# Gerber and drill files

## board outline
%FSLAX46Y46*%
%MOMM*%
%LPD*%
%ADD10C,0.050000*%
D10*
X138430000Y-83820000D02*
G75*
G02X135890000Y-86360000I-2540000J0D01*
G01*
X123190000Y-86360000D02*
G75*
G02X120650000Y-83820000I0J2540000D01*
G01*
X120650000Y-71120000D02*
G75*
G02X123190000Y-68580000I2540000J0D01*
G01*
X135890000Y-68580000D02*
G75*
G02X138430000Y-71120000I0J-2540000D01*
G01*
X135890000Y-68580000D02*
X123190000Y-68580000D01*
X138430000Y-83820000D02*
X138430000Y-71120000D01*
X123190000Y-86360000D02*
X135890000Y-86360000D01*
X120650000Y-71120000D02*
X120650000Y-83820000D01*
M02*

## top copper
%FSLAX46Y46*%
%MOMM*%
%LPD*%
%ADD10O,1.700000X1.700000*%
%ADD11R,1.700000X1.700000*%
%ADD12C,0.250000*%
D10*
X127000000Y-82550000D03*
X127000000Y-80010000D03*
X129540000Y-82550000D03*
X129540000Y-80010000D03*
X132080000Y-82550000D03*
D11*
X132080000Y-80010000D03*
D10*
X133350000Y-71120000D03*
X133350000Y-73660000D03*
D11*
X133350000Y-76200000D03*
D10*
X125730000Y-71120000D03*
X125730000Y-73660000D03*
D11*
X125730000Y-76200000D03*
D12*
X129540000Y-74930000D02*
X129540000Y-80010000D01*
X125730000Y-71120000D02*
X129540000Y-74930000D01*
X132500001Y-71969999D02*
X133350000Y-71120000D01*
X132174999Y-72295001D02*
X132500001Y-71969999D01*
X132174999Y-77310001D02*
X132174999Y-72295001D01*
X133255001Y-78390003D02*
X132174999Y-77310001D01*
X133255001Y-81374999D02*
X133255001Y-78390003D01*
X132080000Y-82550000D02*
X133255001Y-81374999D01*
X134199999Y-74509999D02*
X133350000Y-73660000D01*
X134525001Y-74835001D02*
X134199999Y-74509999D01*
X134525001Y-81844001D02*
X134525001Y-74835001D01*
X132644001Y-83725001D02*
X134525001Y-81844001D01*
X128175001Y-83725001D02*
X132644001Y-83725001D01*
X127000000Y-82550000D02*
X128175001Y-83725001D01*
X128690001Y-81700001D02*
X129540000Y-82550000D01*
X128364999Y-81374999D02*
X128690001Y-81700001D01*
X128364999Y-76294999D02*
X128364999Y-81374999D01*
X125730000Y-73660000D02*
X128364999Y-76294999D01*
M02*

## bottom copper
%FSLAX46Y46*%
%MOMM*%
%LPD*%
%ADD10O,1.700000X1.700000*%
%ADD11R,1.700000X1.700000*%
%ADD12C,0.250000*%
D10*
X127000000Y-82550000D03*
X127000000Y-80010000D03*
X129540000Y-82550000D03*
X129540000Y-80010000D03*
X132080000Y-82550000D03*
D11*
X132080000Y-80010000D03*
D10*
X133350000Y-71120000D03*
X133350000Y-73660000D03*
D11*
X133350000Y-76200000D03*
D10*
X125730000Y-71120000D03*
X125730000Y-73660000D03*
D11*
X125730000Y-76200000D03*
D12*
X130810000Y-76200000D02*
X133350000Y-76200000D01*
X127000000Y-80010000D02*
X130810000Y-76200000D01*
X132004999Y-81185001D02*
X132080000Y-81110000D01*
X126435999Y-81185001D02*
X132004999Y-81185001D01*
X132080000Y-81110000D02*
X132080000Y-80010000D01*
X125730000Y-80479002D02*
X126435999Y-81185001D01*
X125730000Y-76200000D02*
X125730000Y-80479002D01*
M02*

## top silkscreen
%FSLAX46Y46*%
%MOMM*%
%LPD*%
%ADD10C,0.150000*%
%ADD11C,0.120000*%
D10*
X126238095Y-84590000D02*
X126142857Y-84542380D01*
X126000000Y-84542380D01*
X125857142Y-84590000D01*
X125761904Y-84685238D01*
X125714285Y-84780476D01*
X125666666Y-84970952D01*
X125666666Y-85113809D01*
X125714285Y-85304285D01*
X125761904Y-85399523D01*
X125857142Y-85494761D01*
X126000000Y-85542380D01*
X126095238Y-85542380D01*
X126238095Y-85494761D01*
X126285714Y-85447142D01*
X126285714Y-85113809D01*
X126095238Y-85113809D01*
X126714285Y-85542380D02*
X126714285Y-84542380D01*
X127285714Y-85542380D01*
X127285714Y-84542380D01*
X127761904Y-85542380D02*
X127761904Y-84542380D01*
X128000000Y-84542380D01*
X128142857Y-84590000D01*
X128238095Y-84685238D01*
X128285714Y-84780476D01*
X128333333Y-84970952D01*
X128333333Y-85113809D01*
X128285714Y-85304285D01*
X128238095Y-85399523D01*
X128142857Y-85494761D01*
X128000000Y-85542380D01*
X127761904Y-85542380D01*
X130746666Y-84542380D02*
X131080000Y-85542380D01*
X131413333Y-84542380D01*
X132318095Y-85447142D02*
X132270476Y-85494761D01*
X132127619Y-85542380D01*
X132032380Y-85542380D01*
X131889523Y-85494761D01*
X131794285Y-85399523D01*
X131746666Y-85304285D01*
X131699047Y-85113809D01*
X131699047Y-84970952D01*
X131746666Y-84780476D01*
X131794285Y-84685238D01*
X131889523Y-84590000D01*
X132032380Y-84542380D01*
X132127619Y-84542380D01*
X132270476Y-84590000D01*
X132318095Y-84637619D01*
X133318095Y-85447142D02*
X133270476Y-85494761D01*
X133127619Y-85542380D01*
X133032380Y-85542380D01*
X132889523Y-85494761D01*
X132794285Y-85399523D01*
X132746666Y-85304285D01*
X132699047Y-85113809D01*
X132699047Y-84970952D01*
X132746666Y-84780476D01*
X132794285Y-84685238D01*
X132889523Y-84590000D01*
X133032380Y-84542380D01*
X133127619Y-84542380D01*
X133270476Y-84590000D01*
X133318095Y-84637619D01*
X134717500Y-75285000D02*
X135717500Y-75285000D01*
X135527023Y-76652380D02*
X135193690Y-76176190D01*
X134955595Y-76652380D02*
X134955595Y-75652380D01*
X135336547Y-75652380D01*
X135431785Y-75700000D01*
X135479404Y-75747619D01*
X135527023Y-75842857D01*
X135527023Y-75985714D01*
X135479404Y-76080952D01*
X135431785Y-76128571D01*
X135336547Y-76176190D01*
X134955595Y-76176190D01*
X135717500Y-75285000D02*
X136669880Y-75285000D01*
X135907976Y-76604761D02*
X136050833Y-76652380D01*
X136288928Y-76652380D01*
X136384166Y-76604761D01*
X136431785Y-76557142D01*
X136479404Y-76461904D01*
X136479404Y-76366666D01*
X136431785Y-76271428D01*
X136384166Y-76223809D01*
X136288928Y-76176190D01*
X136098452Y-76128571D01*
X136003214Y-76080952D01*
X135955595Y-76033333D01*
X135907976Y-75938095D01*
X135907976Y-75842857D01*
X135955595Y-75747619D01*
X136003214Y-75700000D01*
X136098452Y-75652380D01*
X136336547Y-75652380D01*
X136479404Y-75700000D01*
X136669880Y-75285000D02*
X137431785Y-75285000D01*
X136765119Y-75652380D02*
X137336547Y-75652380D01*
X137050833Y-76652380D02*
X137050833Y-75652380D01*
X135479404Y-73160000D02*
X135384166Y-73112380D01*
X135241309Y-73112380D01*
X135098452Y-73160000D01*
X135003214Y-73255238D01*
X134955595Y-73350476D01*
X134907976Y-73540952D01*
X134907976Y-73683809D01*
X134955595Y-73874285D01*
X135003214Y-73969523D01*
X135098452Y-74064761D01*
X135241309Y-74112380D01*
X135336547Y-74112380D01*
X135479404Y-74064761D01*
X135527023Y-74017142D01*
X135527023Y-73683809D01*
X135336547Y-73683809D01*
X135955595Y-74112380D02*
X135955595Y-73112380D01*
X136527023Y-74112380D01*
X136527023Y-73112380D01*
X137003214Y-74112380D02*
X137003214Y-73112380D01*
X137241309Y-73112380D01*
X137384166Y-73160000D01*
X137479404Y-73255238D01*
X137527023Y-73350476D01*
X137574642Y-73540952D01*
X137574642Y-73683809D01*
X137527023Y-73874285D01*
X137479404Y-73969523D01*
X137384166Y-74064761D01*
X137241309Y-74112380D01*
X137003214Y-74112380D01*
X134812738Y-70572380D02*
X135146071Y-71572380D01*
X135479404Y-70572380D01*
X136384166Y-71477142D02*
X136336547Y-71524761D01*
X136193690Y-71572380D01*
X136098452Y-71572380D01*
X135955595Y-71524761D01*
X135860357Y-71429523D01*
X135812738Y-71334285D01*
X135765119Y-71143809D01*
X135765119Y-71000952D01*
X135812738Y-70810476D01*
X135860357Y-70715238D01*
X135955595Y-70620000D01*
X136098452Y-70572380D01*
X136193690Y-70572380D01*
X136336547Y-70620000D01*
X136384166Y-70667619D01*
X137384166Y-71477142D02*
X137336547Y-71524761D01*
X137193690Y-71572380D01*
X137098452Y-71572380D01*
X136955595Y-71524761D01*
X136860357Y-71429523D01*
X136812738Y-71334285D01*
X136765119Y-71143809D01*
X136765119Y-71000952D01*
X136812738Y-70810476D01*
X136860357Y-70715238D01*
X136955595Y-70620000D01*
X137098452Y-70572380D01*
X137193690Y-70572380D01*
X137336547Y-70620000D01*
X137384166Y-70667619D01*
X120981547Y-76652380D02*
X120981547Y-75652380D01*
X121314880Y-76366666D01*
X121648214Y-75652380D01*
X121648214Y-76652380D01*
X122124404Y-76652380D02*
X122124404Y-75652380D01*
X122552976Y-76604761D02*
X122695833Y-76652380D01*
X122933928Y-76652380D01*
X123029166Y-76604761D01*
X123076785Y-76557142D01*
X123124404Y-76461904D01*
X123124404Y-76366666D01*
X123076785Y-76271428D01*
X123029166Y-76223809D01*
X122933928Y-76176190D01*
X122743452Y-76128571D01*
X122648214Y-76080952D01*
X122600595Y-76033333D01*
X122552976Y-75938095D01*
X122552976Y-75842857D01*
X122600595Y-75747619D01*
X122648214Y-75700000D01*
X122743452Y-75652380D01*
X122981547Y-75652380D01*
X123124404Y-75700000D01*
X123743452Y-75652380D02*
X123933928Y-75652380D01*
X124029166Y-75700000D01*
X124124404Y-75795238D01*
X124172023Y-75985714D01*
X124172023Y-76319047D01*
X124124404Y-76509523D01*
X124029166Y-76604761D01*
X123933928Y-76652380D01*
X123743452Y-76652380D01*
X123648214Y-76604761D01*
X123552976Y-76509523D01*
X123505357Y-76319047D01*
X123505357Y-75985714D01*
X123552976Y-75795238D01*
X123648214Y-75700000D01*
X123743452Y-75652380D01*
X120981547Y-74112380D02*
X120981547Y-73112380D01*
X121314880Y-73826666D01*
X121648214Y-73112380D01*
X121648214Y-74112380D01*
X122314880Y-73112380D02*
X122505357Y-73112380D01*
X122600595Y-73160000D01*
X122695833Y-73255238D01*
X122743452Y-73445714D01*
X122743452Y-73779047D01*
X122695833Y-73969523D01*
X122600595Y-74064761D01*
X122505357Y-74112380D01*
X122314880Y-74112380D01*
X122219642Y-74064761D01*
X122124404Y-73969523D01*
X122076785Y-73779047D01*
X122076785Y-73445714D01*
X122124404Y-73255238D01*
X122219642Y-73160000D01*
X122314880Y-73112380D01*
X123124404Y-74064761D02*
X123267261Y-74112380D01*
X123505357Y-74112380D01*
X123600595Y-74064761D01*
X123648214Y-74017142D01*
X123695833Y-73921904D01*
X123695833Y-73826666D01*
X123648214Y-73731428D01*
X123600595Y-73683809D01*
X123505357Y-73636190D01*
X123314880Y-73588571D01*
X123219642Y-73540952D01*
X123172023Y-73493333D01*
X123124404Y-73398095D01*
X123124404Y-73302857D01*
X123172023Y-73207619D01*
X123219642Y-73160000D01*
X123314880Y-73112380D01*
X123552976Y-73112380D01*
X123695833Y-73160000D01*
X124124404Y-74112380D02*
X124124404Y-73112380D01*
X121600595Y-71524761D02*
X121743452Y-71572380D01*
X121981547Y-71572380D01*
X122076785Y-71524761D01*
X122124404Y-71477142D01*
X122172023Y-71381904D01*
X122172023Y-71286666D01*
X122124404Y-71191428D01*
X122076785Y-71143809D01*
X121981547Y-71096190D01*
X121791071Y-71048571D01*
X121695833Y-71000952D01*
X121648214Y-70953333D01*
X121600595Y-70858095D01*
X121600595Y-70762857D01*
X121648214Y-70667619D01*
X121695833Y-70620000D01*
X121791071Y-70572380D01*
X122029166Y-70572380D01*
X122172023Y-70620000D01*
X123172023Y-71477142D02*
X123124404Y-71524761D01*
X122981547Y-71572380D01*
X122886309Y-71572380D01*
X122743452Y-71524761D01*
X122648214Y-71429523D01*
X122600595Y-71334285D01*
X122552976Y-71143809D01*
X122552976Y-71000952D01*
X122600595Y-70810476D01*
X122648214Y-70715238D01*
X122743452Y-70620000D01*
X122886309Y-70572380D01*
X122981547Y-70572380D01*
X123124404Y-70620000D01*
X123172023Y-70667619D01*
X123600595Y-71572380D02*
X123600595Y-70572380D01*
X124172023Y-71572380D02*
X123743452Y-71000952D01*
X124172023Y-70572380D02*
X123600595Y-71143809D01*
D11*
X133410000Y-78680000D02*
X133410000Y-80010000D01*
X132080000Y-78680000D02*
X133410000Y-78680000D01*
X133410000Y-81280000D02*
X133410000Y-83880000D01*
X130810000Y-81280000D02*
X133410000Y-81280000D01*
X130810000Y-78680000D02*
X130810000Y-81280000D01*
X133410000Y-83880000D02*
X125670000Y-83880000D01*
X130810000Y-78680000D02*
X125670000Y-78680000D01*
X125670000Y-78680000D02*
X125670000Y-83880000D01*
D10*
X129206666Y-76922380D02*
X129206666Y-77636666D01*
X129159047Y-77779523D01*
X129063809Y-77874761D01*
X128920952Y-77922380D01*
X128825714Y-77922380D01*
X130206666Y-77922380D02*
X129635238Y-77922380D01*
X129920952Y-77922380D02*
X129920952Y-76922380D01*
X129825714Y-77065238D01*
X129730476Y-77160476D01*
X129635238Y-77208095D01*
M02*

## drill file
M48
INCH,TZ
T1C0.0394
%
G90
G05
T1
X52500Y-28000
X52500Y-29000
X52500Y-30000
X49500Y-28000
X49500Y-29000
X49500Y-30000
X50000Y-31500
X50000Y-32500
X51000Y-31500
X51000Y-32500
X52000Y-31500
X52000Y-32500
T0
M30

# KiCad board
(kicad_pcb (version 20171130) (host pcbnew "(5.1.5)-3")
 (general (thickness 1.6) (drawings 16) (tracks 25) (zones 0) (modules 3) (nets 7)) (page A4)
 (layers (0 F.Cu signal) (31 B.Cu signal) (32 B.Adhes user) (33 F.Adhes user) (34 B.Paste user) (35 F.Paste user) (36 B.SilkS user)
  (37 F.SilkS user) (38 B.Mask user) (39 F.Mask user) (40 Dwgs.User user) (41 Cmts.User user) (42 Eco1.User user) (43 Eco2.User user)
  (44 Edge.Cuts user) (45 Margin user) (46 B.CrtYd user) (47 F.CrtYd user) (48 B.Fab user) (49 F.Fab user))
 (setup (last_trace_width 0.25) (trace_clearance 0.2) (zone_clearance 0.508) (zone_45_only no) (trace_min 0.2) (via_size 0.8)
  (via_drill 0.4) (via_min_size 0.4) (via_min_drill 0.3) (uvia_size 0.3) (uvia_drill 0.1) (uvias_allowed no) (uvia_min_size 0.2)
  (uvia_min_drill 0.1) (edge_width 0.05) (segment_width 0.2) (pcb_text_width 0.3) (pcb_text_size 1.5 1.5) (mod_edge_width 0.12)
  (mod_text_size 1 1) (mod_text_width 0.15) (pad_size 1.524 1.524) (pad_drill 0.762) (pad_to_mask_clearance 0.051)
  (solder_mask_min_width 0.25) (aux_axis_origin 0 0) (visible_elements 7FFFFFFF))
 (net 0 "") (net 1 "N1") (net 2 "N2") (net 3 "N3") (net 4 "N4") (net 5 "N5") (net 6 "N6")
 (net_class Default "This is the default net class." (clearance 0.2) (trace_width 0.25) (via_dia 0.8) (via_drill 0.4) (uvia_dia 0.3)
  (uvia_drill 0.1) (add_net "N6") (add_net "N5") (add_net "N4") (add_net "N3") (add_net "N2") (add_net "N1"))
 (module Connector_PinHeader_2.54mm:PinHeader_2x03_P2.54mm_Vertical (layer F.Cu) (at 132.08 80.01 270)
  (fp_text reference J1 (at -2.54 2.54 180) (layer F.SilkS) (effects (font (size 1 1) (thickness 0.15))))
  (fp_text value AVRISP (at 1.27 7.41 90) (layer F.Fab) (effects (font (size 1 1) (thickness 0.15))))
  (fp_line (start -1.33 -1.33) (end 0 -1.33) (layer F.SilkS) (width 0.12))
  (fp_line (start -1.33 0) (end -1.33 -1.33) (layer F.SilkS) (width 0.12))
  (fp_line (start 1.27 -1.33) (end 3.87 -1.33) (layer F.SilkS) (width 0.12))
  (fp_line (start 1.27 1.27) (end 1.27 -1.33) (layer F.SilkS) (width 0.12))
  (fp_line (start -1.33 1.27) (end 1.27 1.27) (layer F.SilkS) (width 0.12))
  (fp_line (start 3.87 -1.33) (end 3.87 6.41) (layer F.SilkS) (width 0.12))
  (fp_line (start -1.33 1.27) (end -1.33 6.41) (layer F.SilkS) (width 0.12))
  (fp_line (start -1.33 6.41) (end 3.87 6.41) (layer F.SilkS) (width 0.12))
  (pad 6 thru_hole oval (at 2.54 5.08 270) (size 1.7 1.7) (drill 1) (layers *.Cu *.Mask) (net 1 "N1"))
  (pad 5 thru_hole oval (at 0 5.08 270) (size 1.7 1.7) (drill 1) (layers *.Cu *.Mask) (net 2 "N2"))
  (pad 4 thru_hole oval (at 2.54 2.54 270) (size 1.7 1.7) (drill 1) (layers *.Cu *.Mask) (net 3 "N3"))
  (pad 3 thru_hole oval (at 0 2.54 270) (size 1.7 1.7) (drill 1) (layers *.Cu *.Mask) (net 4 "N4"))
  (pad 2 thru_hole oval (at 2.54 0 270) (size 1.7 1.7) (drill 1) (layers *.Cu *.Mask) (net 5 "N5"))
  (pad 1 thru_hole rect (at 0 0 270) (size 1.7 1.7) (drill 1) (layers *.Cu *.Mask) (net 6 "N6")))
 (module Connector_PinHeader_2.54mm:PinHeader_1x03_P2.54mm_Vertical (layer B.Cu) (at 133.35 76.2)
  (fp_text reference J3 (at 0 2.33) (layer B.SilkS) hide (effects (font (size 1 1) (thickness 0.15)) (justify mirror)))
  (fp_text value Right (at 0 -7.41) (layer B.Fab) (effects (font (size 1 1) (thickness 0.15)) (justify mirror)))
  (pad 3 thru_hole oval (at 0 -5.08) (size 1.7 1.7) (drill 1) (layers *.Cu *.Mask) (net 5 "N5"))
  (pad 2 thru_hole oval (at 0 -2.54) (size 1.7 1.7) (drill 1) (layers *.Cu *.Mask) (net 1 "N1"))
  (pad 1 thru_hole rect (at 0 0) (size 1.7 1.7) (drill 1) (layers *.Cu *.Mask) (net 2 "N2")))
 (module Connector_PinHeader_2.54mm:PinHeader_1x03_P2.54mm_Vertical (layer B.Cu) (at 125.73 76.2)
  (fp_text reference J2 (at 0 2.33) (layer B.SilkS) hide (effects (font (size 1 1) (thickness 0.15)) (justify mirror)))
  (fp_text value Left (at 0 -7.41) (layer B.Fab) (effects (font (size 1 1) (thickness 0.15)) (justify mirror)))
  (pad 3 thru_hole oval (at 0 -5.08) (size 1.7 1.7) (drill 1) (layers *.Cu *.Mask) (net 4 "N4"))
  (pad 2 thru_hole oval (at 0 -2.54) (size 1.7 1.7) (drill 1) (layers *.Cu *.Mask) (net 3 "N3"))
  (pad 1 thru_hole rect (at 0 0) (size 1.7 1.7) (drill 1) (layers *.Cu *.Mask) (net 6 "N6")))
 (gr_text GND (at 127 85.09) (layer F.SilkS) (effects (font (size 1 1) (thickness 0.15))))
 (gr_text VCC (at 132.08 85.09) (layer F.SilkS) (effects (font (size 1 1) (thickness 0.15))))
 (gr_arc (start 135.89 83.82) (end 135.89 86.36) (angle -90) (layer Edge.Cuts) (width 0.05))
 (gr_arc (start 123.19 83.82) (end 120.65 83.82) (angle -90) (layer Edge.Cuts) (width 0.05))
 (gr_arc (start 123.19 71.12) (end 123.19 68.58) (angle -90) (layer Edge.Cuts) (width 0.05))
 (gr_arc (start 135.89 71.12) (end 138.43 71.12) (angle -90) (layer Edge.Cuts) (width 0.05))
 (gr_line (start 135.89 68.58) (end 123.19 68.58) (layer Edge.Cuts) (width 0.05))
 (gr_line (start 138.43 83.82) (end 138.43 71.12) (layer Edge.Cuts) (width 0.05))
 (gr_line (start 123.19 86.36) (end 135.89 86.36) (layer Edge.Cuts) (width 0.05))
 (gr_line (start 120.65 71.12) (end 120.65 83.82) (layer Edge.Cuts) (width 0.05))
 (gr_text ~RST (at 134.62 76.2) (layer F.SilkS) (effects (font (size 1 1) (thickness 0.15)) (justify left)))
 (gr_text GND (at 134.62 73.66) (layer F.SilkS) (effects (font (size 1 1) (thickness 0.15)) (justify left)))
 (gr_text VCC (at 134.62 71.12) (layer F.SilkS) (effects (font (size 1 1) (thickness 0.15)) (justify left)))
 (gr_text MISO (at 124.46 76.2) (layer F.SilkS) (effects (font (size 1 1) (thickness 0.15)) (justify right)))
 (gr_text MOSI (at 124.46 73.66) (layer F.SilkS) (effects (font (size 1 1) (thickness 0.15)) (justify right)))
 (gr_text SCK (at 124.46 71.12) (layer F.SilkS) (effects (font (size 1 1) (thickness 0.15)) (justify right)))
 (segment (start 130.81 76.2) (end 133.35 76.2) (width 0.25) (layer B.Cu) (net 2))
 (segment (start 127 80.01) (end 130.81 76.2) (width 0.25) (layer B.Cu) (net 2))
 (segment (start 129.54 74.93) (end 129.54 80.01) (width 0.25) (layer F.Cu) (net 4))
 (segment (start 125.73 71.12) (end 129.54 74.93) (width 0.25) (layer F.Cu) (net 4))
 (segment (start 132.500001 71.969999) (end 133.35 71.12) (width 0.25) (layer F.Cu) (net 5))
 (segment (start 132.174999 72.295001) (end 132.500001 71.969999) (width 0.25) (layer F.Cu) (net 5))
 (segment (start 132.174999 77.310001) (end 132.174999 72.295001) (width 0.25) (layer F.Cu) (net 5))
 (segment (start 133.255001 78.390003) (end 132.174999 77.310001) (width 0.25) (layer F.Cu) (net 5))
 (segment (start 133.255001 81.374999) (end 133.255001 78.390003) (width 0.25) (layer F.Cu) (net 5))
 (segment (start 132.08 82.55) (end 133.255001 81.374999) (width 0.25) (layer F.Cu) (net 5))
 (segment (start 132.004999 81.185001) (end 132.08 81.11) (width 0.25) (layer B.Cu) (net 6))
 (segment (start 126.435999 81.185001) (end 132.004999 81.185001) (width 0.25) (layer B.Cu) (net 6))
 (segment (start 132.08 81.11) (end 132.08 80.01) (width 0.25) (layer B.Cu) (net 6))
 (segment (start 125.73 80.479002) (end 126.435999 81.185001) (width 0.25) (layer B.Cu) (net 6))
 (segment (start 125.73 76.2) (end 125.73 80.479002) (width 0.25) (layer B.Cu) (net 6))
 (segment (start 134.199999 74.509999) (end 133.35 73.66) (width 0.25) (layer F.Cu) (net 1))
 (segment (start 134.525001 74.835001) (end 134.199999 74.509999) (width 0.25) (layer F.Cu) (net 1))
 (segment (start 134.525001 81.844001) (end 134.525001 74.835001) (width 0.25) (layer F.Cu) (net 1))
 (segment (start 132.644001 83.725001) (end 134.525001 81.844001) (width 0.25) (layer F.Cu) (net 1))
 (segment (start 128.175001 83.725001) (end 132.644001 83.725001) (width 0.25) (layer F.Cu) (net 1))
 (segment (start 127 82.55) (end 128.175001 83.725001) (width 0.25) (layer F.Cu) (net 1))
 (segment (start 128.690001 81.700001) (end 129.54 82.55) (width 0.25) (layer F.Cu) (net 3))
 (segment (start 128.364999 81.374999) (end 128.690001 81.700001) (width 0.25) (layer F.Cu) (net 3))
 (segment (start 128.364999 76.294999) (end 128.364999 81.374999) (width 0.25) (layer F.Cu) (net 3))
 (segment (start 125.73 73.66) (end 128.364999 76.294999) (width 0.25) (layer F.Cu) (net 3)))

